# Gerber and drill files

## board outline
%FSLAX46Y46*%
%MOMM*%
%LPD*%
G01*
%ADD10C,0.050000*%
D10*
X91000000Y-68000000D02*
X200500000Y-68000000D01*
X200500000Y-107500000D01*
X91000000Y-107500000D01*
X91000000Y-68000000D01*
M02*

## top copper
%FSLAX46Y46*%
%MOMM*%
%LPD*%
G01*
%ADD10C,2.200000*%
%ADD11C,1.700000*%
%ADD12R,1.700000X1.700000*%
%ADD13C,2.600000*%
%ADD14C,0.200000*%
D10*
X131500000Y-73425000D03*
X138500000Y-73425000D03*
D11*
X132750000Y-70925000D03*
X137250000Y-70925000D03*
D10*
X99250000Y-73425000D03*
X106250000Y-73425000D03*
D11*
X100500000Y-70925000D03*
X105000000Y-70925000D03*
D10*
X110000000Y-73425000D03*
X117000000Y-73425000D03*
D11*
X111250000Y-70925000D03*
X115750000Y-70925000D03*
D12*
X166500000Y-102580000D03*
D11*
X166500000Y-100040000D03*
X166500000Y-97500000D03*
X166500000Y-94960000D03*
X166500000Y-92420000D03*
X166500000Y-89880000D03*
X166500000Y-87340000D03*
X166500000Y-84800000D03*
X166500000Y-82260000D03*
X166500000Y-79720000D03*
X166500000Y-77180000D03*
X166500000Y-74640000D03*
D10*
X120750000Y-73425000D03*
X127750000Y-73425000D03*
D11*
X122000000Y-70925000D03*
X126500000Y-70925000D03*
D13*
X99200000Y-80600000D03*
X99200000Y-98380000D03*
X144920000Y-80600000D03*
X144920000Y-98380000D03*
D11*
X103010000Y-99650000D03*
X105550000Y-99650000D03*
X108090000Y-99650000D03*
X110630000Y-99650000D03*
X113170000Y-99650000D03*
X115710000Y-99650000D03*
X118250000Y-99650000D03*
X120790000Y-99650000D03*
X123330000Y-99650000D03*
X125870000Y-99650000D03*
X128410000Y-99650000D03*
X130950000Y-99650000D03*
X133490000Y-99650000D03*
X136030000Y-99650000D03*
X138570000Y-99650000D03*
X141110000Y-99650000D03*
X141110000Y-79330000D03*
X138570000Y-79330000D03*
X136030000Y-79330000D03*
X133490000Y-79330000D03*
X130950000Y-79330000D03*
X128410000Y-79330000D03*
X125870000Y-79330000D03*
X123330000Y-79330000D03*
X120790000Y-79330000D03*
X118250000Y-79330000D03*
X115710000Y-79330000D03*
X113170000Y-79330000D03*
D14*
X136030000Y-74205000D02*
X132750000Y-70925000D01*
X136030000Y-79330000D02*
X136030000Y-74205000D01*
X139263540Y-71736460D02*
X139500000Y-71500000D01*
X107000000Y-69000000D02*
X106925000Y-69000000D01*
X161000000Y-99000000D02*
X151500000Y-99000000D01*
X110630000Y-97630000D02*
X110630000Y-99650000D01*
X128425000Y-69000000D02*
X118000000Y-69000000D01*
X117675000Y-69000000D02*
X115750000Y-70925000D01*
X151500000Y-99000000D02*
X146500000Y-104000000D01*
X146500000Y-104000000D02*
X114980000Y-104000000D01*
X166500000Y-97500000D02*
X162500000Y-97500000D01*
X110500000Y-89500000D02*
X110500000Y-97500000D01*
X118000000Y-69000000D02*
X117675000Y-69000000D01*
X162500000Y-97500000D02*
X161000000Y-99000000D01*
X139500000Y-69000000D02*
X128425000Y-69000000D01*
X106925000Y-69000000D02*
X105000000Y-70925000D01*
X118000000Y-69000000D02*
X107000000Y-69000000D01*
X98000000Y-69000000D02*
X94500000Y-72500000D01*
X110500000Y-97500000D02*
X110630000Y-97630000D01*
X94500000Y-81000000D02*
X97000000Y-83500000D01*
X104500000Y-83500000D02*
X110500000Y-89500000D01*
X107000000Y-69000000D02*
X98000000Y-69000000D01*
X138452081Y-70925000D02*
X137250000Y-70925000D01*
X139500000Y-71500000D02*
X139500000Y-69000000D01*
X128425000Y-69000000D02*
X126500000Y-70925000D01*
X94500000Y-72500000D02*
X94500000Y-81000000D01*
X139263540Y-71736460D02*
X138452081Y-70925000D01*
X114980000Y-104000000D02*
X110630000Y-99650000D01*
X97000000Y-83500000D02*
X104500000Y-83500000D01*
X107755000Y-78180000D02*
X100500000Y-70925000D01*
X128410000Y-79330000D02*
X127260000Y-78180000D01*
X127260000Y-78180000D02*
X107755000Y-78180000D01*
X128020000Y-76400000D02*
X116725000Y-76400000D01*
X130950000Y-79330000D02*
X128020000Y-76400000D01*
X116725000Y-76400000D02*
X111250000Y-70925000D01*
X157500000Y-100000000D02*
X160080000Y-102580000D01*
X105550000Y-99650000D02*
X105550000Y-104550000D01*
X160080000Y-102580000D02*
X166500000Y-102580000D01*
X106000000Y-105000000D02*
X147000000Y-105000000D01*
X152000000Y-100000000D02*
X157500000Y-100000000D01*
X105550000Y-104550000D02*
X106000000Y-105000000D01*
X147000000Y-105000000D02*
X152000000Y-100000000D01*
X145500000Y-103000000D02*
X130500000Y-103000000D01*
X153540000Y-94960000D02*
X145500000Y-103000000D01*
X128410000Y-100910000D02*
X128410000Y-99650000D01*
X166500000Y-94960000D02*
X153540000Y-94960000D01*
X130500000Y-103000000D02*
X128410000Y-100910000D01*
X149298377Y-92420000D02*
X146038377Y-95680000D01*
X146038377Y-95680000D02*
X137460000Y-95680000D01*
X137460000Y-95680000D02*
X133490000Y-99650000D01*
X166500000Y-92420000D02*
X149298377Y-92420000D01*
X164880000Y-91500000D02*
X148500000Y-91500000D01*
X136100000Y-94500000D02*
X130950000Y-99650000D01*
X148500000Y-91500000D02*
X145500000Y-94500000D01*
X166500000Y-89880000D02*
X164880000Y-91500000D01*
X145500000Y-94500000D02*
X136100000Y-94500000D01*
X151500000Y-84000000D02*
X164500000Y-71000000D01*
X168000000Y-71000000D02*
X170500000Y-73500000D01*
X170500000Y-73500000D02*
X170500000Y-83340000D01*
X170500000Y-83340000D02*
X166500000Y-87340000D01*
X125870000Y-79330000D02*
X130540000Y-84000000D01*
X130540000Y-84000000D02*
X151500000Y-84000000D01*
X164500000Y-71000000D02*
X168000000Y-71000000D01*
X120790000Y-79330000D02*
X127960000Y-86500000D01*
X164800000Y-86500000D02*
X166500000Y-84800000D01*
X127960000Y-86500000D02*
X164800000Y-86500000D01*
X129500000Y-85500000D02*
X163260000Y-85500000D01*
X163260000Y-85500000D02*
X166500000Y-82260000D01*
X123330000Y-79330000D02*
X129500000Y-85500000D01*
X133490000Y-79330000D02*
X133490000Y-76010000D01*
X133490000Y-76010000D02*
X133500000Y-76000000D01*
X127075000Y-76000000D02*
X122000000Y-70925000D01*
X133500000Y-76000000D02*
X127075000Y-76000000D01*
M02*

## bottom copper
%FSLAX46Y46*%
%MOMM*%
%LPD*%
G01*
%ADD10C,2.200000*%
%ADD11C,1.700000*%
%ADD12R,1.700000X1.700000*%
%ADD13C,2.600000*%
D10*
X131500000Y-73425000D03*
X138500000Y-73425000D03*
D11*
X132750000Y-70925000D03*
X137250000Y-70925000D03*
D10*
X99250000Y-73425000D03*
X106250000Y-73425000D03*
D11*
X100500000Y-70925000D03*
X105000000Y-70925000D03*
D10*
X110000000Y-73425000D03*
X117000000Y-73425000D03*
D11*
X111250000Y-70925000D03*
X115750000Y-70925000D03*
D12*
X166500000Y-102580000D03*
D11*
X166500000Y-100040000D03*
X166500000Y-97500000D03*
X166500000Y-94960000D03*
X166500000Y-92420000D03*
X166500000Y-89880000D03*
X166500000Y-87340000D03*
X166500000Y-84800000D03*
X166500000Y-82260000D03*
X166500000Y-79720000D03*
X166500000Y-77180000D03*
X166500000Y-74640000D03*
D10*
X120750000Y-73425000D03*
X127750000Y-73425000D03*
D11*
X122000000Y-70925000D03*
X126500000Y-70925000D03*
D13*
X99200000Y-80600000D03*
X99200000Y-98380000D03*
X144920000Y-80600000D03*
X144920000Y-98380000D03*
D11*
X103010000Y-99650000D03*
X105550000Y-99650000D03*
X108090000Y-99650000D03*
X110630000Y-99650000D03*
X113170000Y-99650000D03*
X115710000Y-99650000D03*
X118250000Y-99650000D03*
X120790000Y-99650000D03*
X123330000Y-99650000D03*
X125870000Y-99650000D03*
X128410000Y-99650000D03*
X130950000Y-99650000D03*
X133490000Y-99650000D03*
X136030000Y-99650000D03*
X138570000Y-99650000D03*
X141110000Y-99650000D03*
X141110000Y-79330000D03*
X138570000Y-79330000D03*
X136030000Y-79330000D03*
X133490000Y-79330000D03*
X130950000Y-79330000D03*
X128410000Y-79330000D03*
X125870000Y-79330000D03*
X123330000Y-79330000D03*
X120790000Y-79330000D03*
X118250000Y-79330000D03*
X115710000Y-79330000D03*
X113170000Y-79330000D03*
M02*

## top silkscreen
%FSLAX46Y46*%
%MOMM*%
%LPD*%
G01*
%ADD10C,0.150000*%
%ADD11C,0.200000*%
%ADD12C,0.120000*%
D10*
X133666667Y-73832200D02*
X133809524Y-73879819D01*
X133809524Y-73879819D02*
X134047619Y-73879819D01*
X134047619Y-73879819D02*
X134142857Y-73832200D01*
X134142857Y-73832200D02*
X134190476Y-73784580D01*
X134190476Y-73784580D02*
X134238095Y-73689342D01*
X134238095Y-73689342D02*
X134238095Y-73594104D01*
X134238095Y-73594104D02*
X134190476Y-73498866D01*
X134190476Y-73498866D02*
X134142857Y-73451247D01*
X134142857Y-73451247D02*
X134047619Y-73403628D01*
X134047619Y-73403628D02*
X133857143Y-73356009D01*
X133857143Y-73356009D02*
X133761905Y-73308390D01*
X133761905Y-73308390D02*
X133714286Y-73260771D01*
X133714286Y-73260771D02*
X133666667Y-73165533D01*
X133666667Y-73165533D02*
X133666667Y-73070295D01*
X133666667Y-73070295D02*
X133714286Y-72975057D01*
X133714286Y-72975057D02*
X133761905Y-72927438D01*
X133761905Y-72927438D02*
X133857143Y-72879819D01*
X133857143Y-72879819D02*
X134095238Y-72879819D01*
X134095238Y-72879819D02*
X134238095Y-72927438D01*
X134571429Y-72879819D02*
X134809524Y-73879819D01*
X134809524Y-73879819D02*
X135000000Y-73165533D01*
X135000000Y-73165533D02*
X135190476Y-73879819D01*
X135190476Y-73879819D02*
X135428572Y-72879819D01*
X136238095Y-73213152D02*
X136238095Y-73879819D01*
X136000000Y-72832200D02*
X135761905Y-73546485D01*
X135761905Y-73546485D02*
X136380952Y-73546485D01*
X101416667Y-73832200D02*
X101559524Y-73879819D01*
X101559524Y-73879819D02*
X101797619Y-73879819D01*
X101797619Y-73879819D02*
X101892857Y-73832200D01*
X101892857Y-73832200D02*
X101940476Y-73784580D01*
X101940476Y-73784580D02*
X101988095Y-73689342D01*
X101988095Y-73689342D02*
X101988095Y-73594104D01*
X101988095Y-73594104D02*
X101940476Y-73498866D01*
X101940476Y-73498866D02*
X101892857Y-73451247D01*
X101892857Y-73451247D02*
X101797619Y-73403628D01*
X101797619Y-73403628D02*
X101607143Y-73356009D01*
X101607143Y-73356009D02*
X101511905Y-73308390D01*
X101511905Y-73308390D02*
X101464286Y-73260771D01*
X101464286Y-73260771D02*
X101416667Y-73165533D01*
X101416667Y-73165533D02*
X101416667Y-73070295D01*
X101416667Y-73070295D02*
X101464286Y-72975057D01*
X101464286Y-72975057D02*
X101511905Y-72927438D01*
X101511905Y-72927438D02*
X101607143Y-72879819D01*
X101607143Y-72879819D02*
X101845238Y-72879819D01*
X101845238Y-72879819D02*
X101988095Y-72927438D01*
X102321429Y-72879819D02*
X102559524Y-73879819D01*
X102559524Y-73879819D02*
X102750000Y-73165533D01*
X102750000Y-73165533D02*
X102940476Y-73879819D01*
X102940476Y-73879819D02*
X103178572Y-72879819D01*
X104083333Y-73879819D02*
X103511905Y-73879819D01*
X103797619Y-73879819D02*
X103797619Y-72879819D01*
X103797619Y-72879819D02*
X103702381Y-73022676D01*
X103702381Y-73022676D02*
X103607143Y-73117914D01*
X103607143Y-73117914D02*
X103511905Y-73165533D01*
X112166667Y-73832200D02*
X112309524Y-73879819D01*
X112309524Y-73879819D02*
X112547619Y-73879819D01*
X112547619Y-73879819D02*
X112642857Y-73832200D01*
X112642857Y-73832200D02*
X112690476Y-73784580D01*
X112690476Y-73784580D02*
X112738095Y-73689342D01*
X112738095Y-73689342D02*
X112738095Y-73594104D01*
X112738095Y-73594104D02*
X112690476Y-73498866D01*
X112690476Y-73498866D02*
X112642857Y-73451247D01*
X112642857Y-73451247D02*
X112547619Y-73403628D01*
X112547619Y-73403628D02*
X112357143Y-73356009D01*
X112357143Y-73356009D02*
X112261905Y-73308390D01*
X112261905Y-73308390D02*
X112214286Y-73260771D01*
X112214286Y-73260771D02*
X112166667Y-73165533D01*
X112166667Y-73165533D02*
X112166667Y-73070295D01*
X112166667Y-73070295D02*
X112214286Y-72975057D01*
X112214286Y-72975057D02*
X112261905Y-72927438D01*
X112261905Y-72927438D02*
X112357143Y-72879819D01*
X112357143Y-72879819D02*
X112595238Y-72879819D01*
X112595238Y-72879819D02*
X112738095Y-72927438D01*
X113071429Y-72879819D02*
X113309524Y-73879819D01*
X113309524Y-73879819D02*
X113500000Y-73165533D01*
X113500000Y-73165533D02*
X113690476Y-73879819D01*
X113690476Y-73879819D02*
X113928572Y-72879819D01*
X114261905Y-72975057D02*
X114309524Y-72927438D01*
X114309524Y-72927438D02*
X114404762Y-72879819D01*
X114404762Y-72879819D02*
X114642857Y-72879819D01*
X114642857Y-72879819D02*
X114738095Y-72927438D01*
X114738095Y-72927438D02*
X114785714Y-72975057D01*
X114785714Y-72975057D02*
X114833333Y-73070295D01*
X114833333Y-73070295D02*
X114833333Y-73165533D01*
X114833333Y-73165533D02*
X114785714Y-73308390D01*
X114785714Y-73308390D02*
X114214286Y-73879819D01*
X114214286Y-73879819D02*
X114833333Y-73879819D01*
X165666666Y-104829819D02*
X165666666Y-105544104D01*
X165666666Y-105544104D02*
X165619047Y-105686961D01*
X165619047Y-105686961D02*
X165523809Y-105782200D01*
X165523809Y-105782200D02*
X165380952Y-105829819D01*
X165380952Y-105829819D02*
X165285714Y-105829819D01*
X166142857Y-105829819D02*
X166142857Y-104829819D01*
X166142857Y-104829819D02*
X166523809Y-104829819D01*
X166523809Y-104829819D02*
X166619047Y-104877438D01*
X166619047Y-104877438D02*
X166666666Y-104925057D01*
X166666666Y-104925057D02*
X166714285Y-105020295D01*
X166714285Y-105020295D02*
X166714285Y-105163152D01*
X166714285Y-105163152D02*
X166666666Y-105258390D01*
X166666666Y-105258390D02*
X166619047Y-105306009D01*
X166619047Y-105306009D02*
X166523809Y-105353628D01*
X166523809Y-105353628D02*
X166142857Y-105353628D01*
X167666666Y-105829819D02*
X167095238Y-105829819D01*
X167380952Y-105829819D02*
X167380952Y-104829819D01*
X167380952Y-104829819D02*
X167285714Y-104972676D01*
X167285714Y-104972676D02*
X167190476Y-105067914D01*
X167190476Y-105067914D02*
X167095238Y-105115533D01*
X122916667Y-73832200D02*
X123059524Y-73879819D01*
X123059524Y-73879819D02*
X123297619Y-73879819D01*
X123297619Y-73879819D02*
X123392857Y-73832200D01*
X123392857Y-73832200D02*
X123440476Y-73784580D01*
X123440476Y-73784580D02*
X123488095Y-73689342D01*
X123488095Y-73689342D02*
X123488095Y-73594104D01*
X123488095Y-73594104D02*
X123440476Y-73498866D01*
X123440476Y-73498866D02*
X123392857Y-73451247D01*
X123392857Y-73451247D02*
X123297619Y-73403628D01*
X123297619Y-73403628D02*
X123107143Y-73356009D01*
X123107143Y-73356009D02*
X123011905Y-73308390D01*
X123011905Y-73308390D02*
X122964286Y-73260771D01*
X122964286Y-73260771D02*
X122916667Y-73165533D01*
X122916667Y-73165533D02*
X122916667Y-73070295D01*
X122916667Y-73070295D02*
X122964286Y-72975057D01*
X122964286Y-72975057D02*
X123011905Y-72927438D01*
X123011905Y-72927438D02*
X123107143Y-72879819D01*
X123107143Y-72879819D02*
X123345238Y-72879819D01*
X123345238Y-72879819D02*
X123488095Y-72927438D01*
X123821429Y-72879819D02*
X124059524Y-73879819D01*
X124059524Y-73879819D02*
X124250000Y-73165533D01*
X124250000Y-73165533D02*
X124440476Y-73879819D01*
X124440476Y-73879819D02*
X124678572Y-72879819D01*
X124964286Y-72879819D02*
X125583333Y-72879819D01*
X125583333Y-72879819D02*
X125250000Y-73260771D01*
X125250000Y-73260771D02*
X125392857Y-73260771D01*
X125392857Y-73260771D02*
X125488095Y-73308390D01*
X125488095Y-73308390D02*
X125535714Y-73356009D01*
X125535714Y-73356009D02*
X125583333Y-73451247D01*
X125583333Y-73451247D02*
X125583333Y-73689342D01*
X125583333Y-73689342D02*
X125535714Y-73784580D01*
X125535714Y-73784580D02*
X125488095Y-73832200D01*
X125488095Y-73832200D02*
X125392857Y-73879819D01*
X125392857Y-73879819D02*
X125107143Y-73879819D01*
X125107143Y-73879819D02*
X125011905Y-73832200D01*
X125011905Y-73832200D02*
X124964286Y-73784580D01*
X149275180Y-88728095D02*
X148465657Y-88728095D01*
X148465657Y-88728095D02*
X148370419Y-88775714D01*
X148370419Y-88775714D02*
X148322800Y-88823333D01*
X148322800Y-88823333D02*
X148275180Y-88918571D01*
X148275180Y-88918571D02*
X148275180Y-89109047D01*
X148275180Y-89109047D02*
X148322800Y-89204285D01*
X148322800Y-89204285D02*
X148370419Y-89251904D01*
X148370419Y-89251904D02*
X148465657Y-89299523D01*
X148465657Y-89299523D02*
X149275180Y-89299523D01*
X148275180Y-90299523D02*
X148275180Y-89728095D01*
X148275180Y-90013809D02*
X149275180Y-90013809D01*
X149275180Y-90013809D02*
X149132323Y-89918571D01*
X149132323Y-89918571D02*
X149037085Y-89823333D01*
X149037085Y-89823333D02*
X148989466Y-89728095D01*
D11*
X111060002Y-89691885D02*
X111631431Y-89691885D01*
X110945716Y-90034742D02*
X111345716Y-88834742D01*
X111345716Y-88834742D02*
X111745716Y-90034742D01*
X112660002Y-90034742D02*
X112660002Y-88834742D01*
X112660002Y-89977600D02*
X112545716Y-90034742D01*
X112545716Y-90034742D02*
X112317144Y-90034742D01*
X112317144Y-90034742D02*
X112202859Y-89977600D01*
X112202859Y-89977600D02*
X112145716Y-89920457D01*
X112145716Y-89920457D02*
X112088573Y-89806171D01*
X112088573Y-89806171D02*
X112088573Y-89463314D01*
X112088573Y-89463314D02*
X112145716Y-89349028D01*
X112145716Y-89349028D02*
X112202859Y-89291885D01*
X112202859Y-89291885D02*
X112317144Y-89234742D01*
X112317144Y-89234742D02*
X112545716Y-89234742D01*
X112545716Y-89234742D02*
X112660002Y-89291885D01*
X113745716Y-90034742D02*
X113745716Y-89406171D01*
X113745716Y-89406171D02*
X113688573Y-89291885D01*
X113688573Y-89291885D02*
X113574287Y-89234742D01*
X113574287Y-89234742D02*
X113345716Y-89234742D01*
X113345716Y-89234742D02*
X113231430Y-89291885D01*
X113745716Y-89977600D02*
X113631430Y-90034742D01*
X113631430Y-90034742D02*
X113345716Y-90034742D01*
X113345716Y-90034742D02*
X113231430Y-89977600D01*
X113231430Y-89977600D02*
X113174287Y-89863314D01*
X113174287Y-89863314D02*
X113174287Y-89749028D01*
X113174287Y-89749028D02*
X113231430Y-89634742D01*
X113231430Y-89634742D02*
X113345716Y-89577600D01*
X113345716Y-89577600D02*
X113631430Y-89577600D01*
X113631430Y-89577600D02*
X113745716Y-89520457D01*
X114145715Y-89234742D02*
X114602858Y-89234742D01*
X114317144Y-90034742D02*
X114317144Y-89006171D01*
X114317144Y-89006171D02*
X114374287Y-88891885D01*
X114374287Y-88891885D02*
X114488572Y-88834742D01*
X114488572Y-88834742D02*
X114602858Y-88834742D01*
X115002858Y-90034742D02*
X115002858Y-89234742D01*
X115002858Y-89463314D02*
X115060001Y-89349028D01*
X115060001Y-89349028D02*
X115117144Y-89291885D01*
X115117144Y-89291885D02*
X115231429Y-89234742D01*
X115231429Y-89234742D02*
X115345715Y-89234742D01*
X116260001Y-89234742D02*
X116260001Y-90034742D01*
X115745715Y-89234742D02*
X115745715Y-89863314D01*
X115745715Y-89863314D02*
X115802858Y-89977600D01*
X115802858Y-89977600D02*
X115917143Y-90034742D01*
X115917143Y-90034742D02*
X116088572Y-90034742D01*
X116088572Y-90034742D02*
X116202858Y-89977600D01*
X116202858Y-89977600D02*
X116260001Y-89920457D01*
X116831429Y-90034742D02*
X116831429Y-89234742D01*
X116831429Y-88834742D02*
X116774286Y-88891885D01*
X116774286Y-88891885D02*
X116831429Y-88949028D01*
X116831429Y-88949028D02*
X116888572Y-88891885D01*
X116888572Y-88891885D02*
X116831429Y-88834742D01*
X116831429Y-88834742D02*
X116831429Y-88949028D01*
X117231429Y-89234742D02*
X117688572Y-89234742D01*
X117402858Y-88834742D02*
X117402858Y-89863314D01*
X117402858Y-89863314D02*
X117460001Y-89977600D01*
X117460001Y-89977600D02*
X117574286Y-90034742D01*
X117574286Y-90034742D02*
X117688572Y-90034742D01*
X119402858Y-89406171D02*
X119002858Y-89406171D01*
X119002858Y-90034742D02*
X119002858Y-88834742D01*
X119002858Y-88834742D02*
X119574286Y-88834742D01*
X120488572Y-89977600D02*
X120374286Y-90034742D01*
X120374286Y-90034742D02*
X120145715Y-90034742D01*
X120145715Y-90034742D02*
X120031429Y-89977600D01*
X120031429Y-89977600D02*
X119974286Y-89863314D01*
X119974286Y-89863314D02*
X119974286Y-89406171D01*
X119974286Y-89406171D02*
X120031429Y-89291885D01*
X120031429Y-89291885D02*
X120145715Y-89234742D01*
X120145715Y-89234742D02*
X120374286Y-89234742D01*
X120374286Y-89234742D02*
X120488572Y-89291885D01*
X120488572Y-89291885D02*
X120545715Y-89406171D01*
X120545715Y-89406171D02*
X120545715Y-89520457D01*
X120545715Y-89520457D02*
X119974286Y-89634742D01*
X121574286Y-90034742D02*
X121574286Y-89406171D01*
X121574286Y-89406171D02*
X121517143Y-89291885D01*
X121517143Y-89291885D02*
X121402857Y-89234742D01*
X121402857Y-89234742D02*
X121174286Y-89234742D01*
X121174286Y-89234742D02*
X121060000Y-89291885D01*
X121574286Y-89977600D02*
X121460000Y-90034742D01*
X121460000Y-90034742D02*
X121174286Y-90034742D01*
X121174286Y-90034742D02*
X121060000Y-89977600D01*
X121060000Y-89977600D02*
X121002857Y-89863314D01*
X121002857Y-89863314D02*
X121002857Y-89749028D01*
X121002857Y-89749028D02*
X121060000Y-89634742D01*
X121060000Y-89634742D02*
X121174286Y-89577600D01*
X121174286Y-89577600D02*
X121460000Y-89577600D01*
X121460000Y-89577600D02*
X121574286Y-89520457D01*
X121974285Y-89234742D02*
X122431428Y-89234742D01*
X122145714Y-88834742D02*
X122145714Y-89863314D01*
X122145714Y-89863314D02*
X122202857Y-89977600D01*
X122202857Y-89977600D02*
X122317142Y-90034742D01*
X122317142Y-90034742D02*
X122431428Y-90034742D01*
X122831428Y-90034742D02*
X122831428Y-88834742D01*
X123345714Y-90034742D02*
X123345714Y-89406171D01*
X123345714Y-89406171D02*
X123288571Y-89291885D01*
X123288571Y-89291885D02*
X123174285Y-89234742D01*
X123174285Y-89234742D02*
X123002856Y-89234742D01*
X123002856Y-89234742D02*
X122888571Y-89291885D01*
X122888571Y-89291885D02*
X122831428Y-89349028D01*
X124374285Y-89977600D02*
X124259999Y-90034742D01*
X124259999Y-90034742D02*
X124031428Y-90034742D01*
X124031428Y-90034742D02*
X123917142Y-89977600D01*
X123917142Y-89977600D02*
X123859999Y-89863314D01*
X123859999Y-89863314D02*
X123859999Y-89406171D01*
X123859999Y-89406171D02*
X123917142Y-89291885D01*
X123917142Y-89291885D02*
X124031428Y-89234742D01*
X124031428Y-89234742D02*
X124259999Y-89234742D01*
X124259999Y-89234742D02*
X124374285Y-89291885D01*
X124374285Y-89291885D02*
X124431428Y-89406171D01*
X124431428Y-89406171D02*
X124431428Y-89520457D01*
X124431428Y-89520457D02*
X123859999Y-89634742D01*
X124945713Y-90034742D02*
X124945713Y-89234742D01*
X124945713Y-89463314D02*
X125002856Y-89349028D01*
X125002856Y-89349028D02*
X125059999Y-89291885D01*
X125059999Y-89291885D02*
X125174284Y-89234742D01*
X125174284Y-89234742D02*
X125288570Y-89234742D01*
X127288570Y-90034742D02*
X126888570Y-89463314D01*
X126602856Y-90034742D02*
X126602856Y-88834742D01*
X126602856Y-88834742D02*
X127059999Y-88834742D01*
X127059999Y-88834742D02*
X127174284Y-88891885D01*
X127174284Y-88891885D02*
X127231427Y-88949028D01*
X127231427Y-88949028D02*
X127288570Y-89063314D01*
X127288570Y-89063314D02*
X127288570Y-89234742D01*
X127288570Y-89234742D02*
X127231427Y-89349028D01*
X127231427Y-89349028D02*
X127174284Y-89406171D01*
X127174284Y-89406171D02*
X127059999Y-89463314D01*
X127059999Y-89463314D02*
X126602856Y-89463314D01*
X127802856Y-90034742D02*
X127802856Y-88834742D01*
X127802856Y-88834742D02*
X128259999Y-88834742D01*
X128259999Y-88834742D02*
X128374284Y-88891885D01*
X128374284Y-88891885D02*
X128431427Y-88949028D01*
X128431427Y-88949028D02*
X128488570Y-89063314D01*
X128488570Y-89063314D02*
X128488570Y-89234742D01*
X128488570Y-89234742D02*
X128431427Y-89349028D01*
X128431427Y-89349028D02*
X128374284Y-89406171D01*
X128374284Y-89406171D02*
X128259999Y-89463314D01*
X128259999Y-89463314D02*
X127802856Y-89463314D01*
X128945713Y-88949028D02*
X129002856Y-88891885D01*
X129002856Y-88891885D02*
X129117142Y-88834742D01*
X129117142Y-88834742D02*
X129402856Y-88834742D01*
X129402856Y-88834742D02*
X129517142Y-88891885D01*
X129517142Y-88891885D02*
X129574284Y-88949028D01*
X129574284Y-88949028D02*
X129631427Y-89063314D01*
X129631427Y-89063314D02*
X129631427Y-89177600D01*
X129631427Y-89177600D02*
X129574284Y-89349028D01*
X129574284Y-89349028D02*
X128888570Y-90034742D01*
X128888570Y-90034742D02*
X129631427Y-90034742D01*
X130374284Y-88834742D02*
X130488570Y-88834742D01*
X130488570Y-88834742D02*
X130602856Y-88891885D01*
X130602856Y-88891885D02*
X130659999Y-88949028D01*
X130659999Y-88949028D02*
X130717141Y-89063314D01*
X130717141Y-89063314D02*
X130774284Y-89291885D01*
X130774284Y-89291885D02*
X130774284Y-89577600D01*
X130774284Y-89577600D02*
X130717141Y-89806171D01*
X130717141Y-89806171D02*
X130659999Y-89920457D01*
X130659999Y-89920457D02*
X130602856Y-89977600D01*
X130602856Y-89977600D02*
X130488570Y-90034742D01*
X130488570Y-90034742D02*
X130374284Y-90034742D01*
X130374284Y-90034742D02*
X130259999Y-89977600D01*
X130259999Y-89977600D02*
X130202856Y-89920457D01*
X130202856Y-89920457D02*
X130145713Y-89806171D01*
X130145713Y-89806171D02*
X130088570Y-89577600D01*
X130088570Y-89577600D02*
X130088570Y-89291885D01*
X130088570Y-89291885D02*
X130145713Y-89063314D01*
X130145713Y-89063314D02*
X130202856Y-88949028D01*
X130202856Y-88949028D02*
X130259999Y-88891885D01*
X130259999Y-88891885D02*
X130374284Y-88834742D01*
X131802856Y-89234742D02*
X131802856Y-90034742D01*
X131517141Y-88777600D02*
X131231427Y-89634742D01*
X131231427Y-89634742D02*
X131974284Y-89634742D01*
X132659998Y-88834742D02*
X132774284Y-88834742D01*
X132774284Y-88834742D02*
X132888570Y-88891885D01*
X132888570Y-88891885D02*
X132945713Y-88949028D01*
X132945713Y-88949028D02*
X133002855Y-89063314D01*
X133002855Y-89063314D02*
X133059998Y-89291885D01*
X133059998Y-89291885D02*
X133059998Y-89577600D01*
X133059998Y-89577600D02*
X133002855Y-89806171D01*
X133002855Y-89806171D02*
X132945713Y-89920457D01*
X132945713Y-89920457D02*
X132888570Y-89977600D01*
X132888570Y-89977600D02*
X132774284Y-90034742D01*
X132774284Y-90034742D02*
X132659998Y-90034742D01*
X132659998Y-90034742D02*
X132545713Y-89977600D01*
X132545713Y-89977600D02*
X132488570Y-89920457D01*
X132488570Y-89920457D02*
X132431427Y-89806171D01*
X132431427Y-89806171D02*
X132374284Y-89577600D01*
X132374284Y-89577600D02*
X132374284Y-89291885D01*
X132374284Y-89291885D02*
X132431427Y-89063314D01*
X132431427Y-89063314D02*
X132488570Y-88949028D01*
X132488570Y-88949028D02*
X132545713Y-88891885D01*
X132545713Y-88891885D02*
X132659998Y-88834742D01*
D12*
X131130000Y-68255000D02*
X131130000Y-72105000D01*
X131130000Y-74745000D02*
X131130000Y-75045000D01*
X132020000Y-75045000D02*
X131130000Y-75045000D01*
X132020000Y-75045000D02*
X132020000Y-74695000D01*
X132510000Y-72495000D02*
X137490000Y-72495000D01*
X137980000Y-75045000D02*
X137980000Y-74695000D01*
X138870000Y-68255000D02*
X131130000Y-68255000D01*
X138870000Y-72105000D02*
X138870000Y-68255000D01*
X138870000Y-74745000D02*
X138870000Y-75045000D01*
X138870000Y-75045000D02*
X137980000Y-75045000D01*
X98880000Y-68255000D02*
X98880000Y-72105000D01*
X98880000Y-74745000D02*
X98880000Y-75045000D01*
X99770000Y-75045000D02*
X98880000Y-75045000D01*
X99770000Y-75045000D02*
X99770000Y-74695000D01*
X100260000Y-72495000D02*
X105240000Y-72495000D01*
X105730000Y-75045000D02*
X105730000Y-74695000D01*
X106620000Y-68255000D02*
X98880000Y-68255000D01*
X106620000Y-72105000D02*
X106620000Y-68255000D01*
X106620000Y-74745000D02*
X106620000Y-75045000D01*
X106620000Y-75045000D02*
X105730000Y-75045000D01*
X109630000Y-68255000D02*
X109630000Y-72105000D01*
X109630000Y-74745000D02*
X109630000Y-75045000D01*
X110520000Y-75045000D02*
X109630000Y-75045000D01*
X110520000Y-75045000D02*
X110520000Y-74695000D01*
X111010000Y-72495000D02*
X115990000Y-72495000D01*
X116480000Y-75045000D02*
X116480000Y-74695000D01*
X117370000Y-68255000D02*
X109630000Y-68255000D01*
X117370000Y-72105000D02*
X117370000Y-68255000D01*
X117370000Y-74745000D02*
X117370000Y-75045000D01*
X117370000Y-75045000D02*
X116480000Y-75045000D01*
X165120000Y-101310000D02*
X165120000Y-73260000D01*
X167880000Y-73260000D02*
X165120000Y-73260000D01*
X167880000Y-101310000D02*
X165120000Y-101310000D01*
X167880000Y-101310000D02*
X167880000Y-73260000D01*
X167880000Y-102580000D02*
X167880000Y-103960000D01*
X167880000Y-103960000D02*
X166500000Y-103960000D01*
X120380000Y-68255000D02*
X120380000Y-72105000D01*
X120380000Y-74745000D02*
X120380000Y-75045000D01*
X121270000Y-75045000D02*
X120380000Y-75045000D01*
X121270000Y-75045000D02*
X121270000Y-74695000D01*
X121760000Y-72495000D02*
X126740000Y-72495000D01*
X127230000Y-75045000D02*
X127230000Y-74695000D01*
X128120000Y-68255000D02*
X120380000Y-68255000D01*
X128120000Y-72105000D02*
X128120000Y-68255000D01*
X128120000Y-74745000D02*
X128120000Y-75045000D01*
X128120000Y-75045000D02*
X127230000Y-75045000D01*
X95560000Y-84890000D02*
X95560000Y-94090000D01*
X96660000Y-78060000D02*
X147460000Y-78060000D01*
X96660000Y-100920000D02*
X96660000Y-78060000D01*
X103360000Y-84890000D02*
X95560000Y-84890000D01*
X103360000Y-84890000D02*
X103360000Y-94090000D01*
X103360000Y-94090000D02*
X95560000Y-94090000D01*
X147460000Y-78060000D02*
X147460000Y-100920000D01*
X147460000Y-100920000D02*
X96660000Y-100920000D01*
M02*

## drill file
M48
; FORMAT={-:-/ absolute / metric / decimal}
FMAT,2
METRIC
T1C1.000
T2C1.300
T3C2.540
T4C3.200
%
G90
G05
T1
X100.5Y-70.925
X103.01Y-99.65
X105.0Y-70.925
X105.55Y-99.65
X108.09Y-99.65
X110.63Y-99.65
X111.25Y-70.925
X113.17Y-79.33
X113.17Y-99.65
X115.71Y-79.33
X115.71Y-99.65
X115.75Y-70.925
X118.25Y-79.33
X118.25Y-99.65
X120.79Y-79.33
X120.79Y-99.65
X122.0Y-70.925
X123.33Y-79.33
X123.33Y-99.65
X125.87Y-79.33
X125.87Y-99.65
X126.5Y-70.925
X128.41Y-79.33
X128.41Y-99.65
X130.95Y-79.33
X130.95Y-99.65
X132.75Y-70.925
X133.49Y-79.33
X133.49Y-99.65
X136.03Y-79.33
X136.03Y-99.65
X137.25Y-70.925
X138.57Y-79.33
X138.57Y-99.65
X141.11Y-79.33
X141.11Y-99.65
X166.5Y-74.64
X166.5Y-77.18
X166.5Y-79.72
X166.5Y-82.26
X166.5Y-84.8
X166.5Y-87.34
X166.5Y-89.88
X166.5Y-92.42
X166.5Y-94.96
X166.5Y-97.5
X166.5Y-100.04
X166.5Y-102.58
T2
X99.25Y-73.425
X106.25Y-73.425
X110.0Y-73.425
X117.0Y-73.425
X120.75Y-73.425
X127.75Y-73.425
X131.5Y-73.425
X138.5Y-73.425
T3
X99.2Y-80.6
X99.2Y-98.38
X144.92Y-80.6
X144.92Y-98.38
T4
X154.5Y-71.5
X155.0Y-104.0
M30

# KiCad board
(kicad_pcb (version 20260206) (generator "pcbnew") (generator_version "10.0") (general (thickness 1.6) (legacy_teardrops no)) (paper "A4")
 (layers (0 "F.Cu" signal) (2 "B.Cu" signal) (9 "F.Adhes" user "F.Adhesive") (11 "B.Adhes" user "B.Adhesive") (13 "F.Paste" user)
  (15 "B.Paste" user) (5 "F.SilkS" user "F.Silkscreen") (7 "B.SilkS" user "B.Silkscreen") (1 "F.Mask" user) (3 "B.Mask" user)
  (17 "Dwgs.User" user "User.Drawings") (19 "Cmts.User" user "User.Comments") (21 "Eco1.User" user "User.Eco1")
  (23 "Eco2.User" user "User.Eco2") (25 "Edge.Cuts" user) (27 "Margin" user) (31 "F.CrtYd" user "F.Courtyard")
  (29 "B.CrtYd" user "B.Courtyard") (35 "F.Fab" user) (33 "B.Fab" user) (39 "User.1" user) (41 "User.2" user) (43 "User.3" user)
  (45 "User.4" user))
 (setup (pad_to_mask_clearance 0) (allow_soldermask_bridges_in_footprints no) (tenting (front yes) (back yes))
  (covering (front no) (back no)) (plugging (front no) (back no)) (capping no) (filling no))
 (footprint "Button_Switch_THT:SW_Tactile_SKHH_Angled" (layer "F.Cu") (at 132.75 70.925)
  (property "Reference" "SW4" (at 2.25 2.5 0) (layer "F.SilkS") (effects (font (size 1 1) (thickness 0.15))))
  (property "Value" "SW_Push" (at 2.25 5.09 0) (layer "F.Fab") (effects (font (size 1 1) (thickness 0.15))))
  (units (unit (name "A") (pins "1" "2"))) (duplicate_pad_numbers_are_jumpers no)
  (fp_line (start -1.62 -2.67) (end -1.62 1.18) (stroke (width 0.12) (type solid)) (layer "F.SilkS"))
  (fp_line (start -1.62 3.82) (end -1.62 4.12) (stroke (width 0.12) (type solid)) (layer "F.SilkS"))
  (fp_line (start -0.73 4.12) (end -1.62 4.12) (stroke (width 0.12) (type solid)) (layer "F.SilkS"))
  (fp_line (start -0.73 4.12) (end -0.73 3.77) (stroke (width 0.12) (type solid)) (layer "F.SilkS"))
  (fp_line (start -0.24 1.57) (end 4.74 1.57) (stroke (width 0.12) (type solid)) (layer "F.SilkS"))
  (fp_line (start 5.23 4.12) (end 5.23 3.77) (stroke (width 0.12) (type solid)) (layer "F.SilkS"))
  (fp_line (start 6.12 -2.67) (end -1.62 -2.67) (stroke (width 0.12) (type solid)) (layer "F.SilkS"))
  (fp_line (start 6.12 1.18) (end 6.12 -2.67) (stroke (width 0.12) (type solid)) (layer "F.SilkS"))
  (fp_line (start 6.12 3.82) (end 6.12 4.12) (stroke (width 0.12) (type solid)) (layer "F.SilkS"))
  (fp_line (start 6.12 4.12) (end 5.23 4.12) (stroke (width 0.12) (type solid)) (layer "F.SilkS"))
  (pad "" thru_hole circle (at -1.25 2.5 180) (size 2.2 2.2) (drill 1.3) (layers "*.Cu" "*.Mask") (remove_unused_layers no))
  (pad "" thru_hole circle (at 5.75 2.5 180) (size 2.2 2.2) (drill 1.3) (layers "*.Cu" "*.Mask") (remove_unused_layers no))
  (pad "1" thru_hole circle (at 0 0 180) (size 1.7 1.7) (drill 1) (layers "*.Cu" "*.Mask") (remove_unused_layers no)
   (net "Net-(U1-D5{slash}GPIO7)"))
  (pad "2" thru_hole circle (at 4.5 0 180) (size 1.7 1.7) (drill 1) (layers "*.Cu" "*.Mask") (remove_unused_layers no) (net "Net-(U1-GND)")))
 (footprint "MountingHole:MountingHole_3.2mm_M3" (layer "F.Cu") (at 155 104)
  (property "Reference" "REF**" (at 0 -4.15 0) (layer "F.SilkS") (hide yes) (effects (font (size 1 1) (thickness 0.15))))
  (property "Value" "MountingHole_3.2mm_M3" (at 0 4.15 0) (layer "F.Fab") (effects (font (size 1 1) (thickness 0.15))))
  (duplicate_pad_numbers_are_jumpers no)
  (pad "" np_thru_hole circle (at 0 0) (size 3.2 3.2) (drill 3.2) (layers "*.Cu" "*.Mask")))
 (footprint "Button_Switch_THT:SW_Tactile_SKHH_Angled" (layer "F.Cu") (at 100.5 70.925)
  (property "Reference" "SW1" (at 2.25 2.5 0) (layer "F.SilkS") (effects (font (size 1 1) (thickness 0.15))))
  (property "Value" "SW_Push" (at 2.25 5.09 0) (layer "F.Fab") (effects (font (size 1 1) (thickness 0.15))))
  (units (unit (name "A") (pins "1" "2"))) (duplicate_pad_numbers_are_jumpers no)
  (fp_line (start -1.62 -2.67) (end -1.62 1.18) (stroke (width 0.12) (type solid)) (layer "F.SilkS"))
  (fp_line (start -1.62 3.82) (end -1.62 4.12) (stroke (width 0.12) (type solid)) (layer "F.SilkS"))
  (fp_line (start -0.73 4.12) (end -1.62 4.12) (stroke (width 0.12) (type solid)) (layer "F.SilkS"))
  (fp_line (start -0.73 4.12) (end -0.73 3.77) (stroke (width 0.12) (type solid)) (layer "F.SilkS"))
  (fp_line (start -0.24 1.57) (end 4.74 1.57) (stroke (width 0.12) (type solid)) (layer "F.SilkS"))
  (fp_line (start 5.23 4.12) (end 5.23 3.77) (stroke (width 0.12) (type solid)) (layer "F.SilkS"))
  (fp_line (start 6.12 -2.67) (end -1.62 -2.67) (stroke (width 0.12) (type solid)) (layer "F.SilkS"))
  (fp_line (start 6.12 1.18) (end 6.12 -2.67) (stroke (width 0.12) (type solid)) (layer "F.SilkS"))
  (fp_line (start 6.12 3.82) (end 6.12 4.12) (stroke (width 0.12) (type solid)) (layer "F.SilkS"))
  (fp_line (start 6.12 4.12) (end 5.23 4.12) (stroke (width 0.12) (type solid)) (layer "F.SilkS"))
  (pad "" thru_hole circle (at -1.25 2.5 180) (size 2.2 2.2) (drill 1.3) (layers "*.Cu" "*.Mask") (remove_unused_layers no))
  (pad "" thru_hole circle (at 5.75 2.5 180) (size 2.2 2.2) (drill 1.3) (layers "*.Cu" "*.Mask") (remove_unused_layers no))
  (pad "1" thru_hole circle (at 0 0 180) (size 1.7 1.7) (drill 1) (layers "*.Cu" "*.Mask") (remove_unused_layers no)
   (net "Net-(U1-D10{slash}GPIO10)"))
  (pad "2" thru_hole circle (at 4.5 0 180) (size 1.7 1.7) (drill 1) (layers "*.Cu" "*.Mask") (remove_unused_layers no) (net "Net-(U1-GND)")))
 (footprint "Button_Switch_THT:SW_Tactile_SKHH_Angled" (layer "F.Cu") (at 111.25 70.925)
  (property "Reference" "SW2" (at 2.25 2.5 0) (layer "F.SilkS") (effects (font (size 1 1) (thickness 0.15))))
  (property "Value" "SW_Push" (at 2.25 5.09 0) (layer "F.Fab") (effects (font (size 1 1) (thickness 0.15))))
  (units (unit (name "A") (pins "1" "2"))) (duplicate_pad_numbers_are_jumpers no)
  (fp_line (start -1.62 -2.67) (end -1.62 1.18) (stroke (width 0.12) (type solid)) (layer "F.SilkS"))
  (fp_line (start -1.62 3.82) (end -1.62 4.12) (stroke (width 0.12) (type solid)) (layer "F.SilkS"))
  (fp_line (start -0.73 4.12) (end -1.62 4.12) (stroke (width 0.12) (type solid)) (layer "F.SilkS"))
  (fp_line (start -0.73 4.12) (end -0.73 3.77) (stroke (width 0.12) (type solid)) (layer "F.SilkS"))
  (fp_line (start -0.24 1.57) (end 4.74 1.57) (stroke (width 0.12) (type solid)) (layer "F.SilkS"))
  (fp_line (start 5.23 4.12) (end 5.23 3.77) (stroke (width 0.12) (type solid)) (layer "F.SilkS"))
  (fp_line (start 6.12 -2.67) (end -1.62 -2.67) (stroke (width 0.12) (type solid)) (layer "F.SilkS"))
  (fp_line (start 6.12 1.18) (end 6.12 -2.67) (stroke (width 0.12) (type solid)) (layer "F.SilkS"))
  (fp_line (start 6.12 3.82) (end 6.12 4.12) (stroke (width 0.12) (type solid)) (layer "F.SilkS"))
  (fp_line (start 6.12 4.12) (end 5.23 4.12) (stroke (width 0.12) (type solid)) (layer "F.SilkS"))
  (pad "" thru_hole circle (at -1.25 2.5 180) (size 2.2 2.2) (drill 1.3) (layers "*.Cu" "*.Mask") (remove_unused_layers no))
  (pad "" thru_hole circle (at 5.75 2.5 180) (size 2.2 2.2) (drill 1.3) (layers "*.Cu" "*.Mask") (remove_unused_layers no))
  (pad "1" thru_hole circle (at 0 0 180) (size 1.7 1.7) (drill 1) (layers "*.Cu" "*.Mask") (remove_unused_layers no)
   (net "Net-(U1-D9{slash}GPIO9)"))
  (pad "2" thru_hole circle (at 4.5 0 180) (size 1.7 1.7) (drill 1) (layers "*.Cu" "*.Mask") (remove_unused_layers no) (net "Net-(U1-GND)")))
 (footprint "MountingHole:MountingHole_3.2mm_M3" (layer "F.Cu") (at 154.5 71.5)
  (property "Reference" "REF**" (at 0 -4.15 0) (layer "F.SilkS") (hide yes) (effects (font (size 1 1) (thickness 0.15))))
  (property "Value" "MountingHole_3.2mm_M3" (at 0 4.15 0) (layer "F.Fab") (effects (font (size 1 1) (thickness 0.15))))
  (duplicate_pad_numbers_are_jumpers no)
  (pad "" np_thru_hole circle (at 0 0) (size 3.2 3.2) (drill 3.2) (layers "*.Cu" "*.Mask")))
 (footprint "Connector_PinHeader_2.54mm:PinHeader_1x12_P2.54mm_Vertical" (layer "F.Cu") (at 166.5 102.58 180)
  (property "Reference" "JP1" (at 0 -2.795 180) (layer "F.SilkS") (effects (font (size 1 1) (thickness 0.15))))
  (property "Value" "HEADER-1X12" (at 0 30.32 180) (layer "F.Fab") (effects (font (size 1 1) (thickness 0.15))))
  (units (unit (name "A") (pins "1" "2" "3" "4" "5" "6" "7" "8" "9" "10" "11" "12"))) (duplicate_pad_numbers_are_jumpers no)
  (fp_line (start 1.38 1.27) (end 1.38 29.32) (stroke (width 0.12) (type solid)) (layer "F.SilkS"))
  (fp_line (start -1.38 29.32) (end 1.38 29.32) (stroke (width 0.12) (type solid)) (layer "F.SilkS"))
  (fp_line (start -1.38 1.27) (end 1.38 1.27) (stroke (width 0.12) (type solid)) (layer "F.SilkS"))
  (fp_line (start -1.38 1.27) (end -1.38 29.32) (stroke (width 0.12) (type solid)) (layer "F.SilkS"))
  (fp_line (start -1.38 0) (end -1.38 -1.38) (stroke (width 0.12) (type solid)) (layer "F.SilkS"))
  (fp_line (start -1.38 -1.38) (end 0 -1.38) (stroke (width 0.12) (type solid)) (layer "F.SilkS"))
  (pad "1" thru_hole rect (at 0 0 180) (size 1.7 1.7) (drill 1) (layers "*.Cu" "*.Mask") (remove_unused_layers no) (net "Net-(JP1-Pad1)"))
  (pad "2" thru_hole circle (at 0 2.54 180) (size 1.7 1.7) (drill 1) (layers "*.Cu" "*.Mask") (remove_unused_layers no)
   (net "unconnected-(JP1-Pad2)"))
  (pad "3" thru_hole circle (at 0 5.08 180) (size 1.7 1.7) (drill 1) (layers "*.Cu" "*.Mask") (remove_unused_layers no) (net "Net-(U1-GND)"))
  (pad "4" thru_hole circle (at 0 7.62 180) (size 1.7 1.7) (drill 1) (layers "*.Cu" "*.Mask") (remove_unused_layers no) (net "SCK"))
  (pad "5" thru_hole circle (at 0 10.16 180) (size 1.7 1.7) (drill 1) (layers "*.Cu" "*.Mask") (remove_unused_layers no) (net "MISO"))
  (pad "6" thru_hole circle (at 0 12.7 180) (size 1.7 1.7) (drill 1) (layers "*.Cu" "*.Mask") (remove_unused_layers no) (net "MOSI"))
  (pad "7" thru_hole circle (at 0 15.24 180) (size 1.7 1.7) (drill 1) (layers "*.Cu" "*.Mask") (remove_unused_layers no) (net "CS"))
  (pad "8" thru_hole circle (at 0 17.78 180) (size 1.7 1.7) (drill 1) (layers "*.Cu" "*.Mask") (remove_unused_layers no) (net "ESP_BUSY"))
  (pad "9" thru_hole circle (at 0 20.32 180) (size 1.7 1.7) (drill 1) (layers "*.Cu" "*.Mask") (remove_unused_layers no) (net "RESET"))
  (pad "10" thru_hole circle (at 0 22.86 180) (size 1.7 1.7) (drill 1) (layers "*.Cu" "*.Mask") (remove_unused_layers no) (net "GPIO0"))
  (pad "11" thru_hole circle (at 0 25.4 180) (size 1.7 1.7) (drill 1) (layers "*.Cu" "*.Mask") (remove_unused_layers no) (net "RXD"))
  (pad "12" thru_hole circle (at 0 27.94 180) (size 1.7 1.7) (drill 1) (layers "*.Cu" "*.Mask") (remove_unused_layers no) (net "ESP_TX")))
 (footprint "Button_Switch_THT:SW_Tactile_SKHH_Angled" (layer "F.Cu") (at 122 70.925)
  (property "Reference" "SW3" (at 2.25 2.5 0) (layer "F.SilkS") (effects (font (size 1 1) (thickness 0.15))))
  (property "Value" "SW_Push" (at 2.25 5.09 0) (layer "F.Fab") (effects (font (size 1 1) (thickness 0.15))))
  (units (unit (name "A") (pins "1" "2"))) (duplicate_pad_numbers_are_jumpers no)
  (fp_line (start -1.62 -2.67) (end -1.62 1.18) (stroke (width 0.12) (type solid)) (layer "F.SilkS"))
  (fp_line (start -1.62 3.82) (end -1.62 4.12) (stroke (width 0.12) (type solid)) (layer "F.SilkS"))
  (fp_line (start -0.73 4.12) (end -1.62 4.12) (stroke (width 0.12) (type solid)) (layer "F.SilkS"))
  (fp_line (start -0.73 4.12) (end -0.73 3.77) (stroke (width 0.12) (type solid)) (layer "F.SilkS"))
  (fp_line (start -0.24 1.57) (end 4.74 1.57) (stroke (width 0.12) (type solid)) (layer "F.SilkS"))
  (fp_line (start 5.23 4.12) (end 5.23 3.77) (stroke (width 0.12) (type solid)) (layer "F.SilkS"))
  (fp_line (start 6.12 -2.67) (end -1.62 -2.67) (stroke (width 0.12) (type solid)) (layer "F.SilkS"))
  (fp_line (start 6.12 1.18) (end 6.12 -2.67) (stroke (width 0.12) (type solid)) (layer "F.SilkS"))
  (fp_line (start 6.12 3.82) (end 6.12 4.12) (stroke (width 0.12) (type solid)) (layer "F.SilkS"))
  (fp_line (start 6.12 4.12) (end 5.23 4.12) (stroke (width 0.12) (type solid)) (layer "F.SilkS"))
  (pad "" thru_hole circle (at -1.25 2.5 180) (size 2.2 2.2) (drill 1.3) (layers "*.Cu" "*.Mask") (remove_unused_layers no))
  (pad "" thru_hole circle (at 5.75 2.5 180) (size 2.2 2.2) (drill 1.3) (layers "*.Cu" "*.Mask") (remove_unused_layers no))
  (pad "1" thru_hole circle (at 0 0 180) (size 1.7 1.7) (drill 1) (layers "*.Cu" "*.Mask") (remove_unused_layers no)
   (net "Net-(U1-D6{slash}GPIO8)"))
  (pad "2" thru_hole circle (at 4.5 0 180) (size 1.7 1.7) (drill 1) (layers "*.Cu" "*.Mask") (remove_unused_layers no) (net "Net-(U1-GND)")))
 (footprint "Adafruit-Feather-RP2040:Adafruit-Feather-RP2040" (layer "F.Cu") (at 122.06 89.49)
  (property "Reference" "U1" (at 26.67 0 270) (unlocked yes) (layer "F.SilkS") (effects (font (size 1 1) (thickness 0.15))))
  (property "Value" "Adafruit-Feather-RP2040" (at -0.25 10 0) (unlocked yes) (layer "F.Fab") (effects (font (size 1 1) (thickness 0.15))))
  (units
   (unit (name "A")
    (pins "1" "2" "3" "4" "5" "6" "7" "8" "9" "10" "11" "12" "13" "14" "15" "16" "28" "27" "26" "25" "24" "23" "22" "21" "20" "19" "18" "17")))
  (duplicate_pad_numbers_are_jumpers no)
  (fp_line (start -26.5 -4.6) (end -26.5 4.6) (stroke (width 0.12) (type solid)) (layer "F.SilkS"))
  (fp_line (start -25.4 -11.43) (end 25.4 -11.43) (stroke (width 0.12) (type solid)) (layer "F.SilkS"))
  (fp_line (start -25.4 11.43) (end -25.4 -11.43) (stroke (width 0.12) (type solid)) (layer "F.SilkS"))
  (fp_line (start -18.7 -4.6) (end -26.5 -4.6) (stroke (width 0.12) (type solid)) (layer "F.SilkS"))
  (fp_line (start -18.7 -4.6) (end -18.7 4.6) (stroke (width 0.12) (type solid)) (layer "F.SilkS"))
  (fp_line (start -18.7 4.6) (end -26.5 4.6) (stroke (width 0.12) (type solid)) (layer "F.SilkS"))
  (fp_line (start 25.4 -11.43) (end 25.4 11.43) (stroke (width 0.12) (type solid)) (layer "F.SilkS"))
  (fp_line (start 25.4 11.43) (end -25.4 11.43) (stroke (width 0.12) (type solid)) (layer "F.SilkS"))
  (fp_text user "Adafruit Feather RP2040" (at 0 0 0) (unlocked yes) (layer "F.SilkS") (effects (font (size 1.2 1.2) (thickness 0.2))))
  (pad "" np_thru_hole circle (at -22.86 -8.89) (size 2.6 2.6) (drill 2.54) (layers "*.Cu" "*.Mask") (solder_mask_margin 1.3)
   (clearance 1.3))
  (pad "" np_thru_hole circle (at -22.86 8.89) (size 2.6 2.6) (drill 2.54) (layers "*.Cu" "*.Mask") (solder_mask_margin 1.3) (clearance 1.3))
  (pad "" np_thru_hole circle (at 22.86 -8.89) (size 2.6 2.6) (drill 2.54) (layers "*.Cu" "*.Mask") (solder_mask_margin 1.3) (clearance 1.3))
  (pad "" np_thru_hole circle (at 22.86 8.89) (size 2.6 2.6) (drill 2.54) (layers "*.Cu" "*.Mask") (solder_mask_margin 1.3) (clearance 1.3))
  (pad "1" thru_hole circle (at -19.05 10.16) (size 1.7 1.7) (drill 1) (layers "*.Cu" "*.Mask") (remove_unused_layers no)
   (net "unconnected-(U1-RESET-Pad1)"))
  (pad "2" thru_hole circle (at -16.51 10.16) (size 1.7 1.7) (drill 1) (layers "*.Cu" "*.Mask") (remove_unused_layers no)
   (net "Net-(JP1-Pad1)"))
  (pad "3" thru_hole circle (at -13.97 10.16) (size 1.7 1.7) (drill 1) (layers "*.Cu" "*.Mask") (remove_unused_layers no)
   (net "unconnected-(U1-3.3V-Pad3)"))
  (pad "4" thru_hole circle (at -11.43 10.16) (size 1.7 1.7) (drill 1) (layers "*.Cu" "*.Mask") (remove_unused_layers no)
   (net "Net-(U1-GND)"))
  (pad "5" thru_hole circle (at -8.89 10.16) (size 1.7 1.7) (drill 1) (layers "*.Cu" "*.Mask") (remove_unused_layers no)
   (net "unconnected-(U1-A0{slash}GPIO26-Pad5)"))
  (pad "6" thru_hole circle (at -6.35 10.16) (size 1.7 1.7) (drill 1) (layers "*.Cu" "*.Mask") (remove_unused_layers no)
   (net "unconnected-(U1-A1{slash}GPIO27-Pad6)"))
  (pad "7" thru_hole circle (at -3.81 10.16) (size 1.7 1.7) (drill 1) (layers "*.Cu" "*.Mask") (remove_unused_layers no)
   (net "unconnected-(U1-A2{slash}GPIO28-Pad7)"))
  (pad "8" thru_hole circle (at -1.27 10.16) (size 1.7 1.7) (drill 1) (layers "*.Cu" "*.Mask") (remove_unused_layers no)
   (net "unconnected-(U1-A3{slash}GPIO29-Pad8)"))
  (pad "9" thru_hole circle (at 1.27 10.16) (size 1.7 1.7) (drill 1) (layers "*.Cu" "*.Mask") (remove_unused_layers no)
   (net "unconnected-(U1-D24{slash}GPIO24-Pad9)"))
  (pad "10" thru_hole circle (at 3.81 10.16) (size 1.7 1.7) (drill 1) (layers "*.Cu" "*.Mask") (remove_unused_layers no)
   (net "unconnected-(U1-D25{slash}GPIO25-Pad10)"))
  (pad "11" thru_hole circle (at 6.35 10.16) (size 1.7 1.7) (drill 1) (layers "*.Cu" "*.Mask") (remove_unused_layers no) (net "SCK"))
  (pad "12" thru_hole circle (at 8.89 10.16) (size 1.7 1.7) (drill 1) (layers "*.Cu" "*.Mask") (remove_unused_layers no) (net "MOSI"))
  (pad "13" thru_hole circle (at 11.43 10.16) (size 1.7 1.7) (drill 1) (layers "*.Cu" "*.Mask") (remove_unused_layers no) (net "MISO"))
  (pad "14" thru_hole circle (at 13.97 10.16) (size 1.7 1.7) (drill 1) (layers "*.Cu" "*.Mask") (remove_unused_layers no)
   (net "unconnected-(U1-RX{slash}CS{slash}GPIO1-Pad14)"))
  (pad "15" thru_hole circle (at 16.51 10.16) (size 1.7 1.7) (drill 1) (layers "*.Cu" "*.Mask") (remove_unused_layers no)
   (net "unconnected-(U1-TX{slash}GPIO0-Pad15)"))
  (pad "16" thru_hole circle (at 19.05 10.16) (size 1.7 1.7) (drill 1) (layers "*.Cu" "*.Mask") (remove_unused_layers no)
   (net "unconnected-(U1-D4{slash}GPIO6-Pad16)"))
  (pad "17" thru_hole circle (at 19.05 -10.16) (size 1.7 1.7) (drill 1) (layers "*.Cu" "*.Mask") (remove_unused_layers no)
   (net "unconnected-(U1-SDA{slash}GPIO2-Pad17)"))
  (pad "18" thru_hole circle (at 16.51 -10.16) (size 1.7 1.7) (drill 1) (layers "*.Cu" "*.Mask") (remove_unused_layers no)
   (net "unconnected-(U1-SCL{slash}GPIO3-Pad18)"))
  (pad "19" thru_hole circle (at 13.97 -10.16) (size 1.7 1.7) (drill 1) (layers "*.Cu" "*.Mask") (remove_unused_layers no)
   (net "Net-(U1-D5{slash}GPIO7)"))
  (pad "20" thru_hole circle (at 11.43 -10.16) (size 1.7 1.7) (drill 1) (layers "*.Cu" "*.Mask") (remove_unused_layers no)
   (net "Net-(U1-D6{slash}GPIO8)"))
  (pad "21" thru_hole circle (at 8.89 -10.16) (size 1.7 1.7) (drill 1) (layers "*.Cu" "*.Mask") (remove_unused_layers no)
   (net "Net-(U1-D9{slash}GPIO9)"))
  (pad "22" thru_hole circle (at 6.35 -10.16) (size 1.7 1.7) (drill 1) (layers "*.Cu" "*.Mask") (remove_unused_layers no)
   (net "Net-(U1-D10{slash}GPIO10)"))
  (pad "23" thru_hole circle (at 3.81 -10.16) (size 1.7 1.7) (drill 1) (layers "*.Cu" "*.Mask") (remove_unused_layers no) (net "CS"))
  (pad "24" thru_hole circle (at 1.27 -10.16) (size 1.7 1.7) (drill 1) (layers "*.Cu" "*.Mask") (remove_unused_layers no) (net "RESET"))
  (pad "25" thru_hole circle (at -1.27 -10.16) (size 1.7 1.7) (drill 1) (layers "*.Cu" "*.Mask") (remove_unused_layers no) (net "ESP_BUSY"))
  (pad "26" thru_hole circle (at -3.81 -10.16) (size 1.7 1.7) (drill 1) (layers "*.Cu" "*.Mask") (remove_unused_layers no)
   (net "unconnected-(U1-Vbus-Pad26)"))
  (pad "27" thru_hole circle (at -6.35 -10.16) (size 1.7 1.7) (drill 1) (layers "*.Cu" "*.Mask") (remove_unused_layers no)
   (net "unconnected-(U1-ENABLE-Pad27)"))
  (pad "28" thru_hole circle (at -8.89 -10.16) (size 1.7 1.7) (drill 1) (layers "*.Cu" "*.Mask") (remove_unused_layers no)
   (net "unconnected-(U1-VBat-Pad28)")))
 (gr_rect (start 91 68) (end 200.5 107.5) (stroke (width 0.05) (type default)) (fill no) (layer "Edge.Cuts"))
 (segment (start 136.03 74.205) (end 132.75 70.925) (width 0.2) (layer "F.Cu") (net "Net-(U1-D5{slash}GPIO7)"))
 (segment (start 136.03 79.33) (end 136.03 74.205) (width 0.2) (layer "F.Cu") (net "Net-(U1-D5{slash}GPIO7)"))
 (segment (start 139.26354 71.73646) (end 139.5 71.5) (width 0.2) (layer "F.Cu") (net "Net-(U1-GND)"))
 (segment (start 107 69) (end 106.925 69) (width 0.2) (layer "F.Cu") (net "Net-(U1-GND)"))
 (segment (start 161 99) (end 151.5 99) (width 0.2) (layer "F.Cu") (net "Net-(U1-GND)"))
 (segment (start 110.63 97.63) (end 110.63 99.65) (width 0.2) (layer "F.Cu") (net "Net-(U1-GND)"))
 (segment (start 128.425 69) (end 118 69) (width 0.2) (layer "F.Cu") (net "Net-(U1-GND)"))
 (segment (start 117.675 69) (end 115.75 70.925) (width 0.2) (layer "F.Cu") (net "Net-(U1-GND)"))
 (segment (start 151.5 99) (end 146.5 104) (width 0.2) (layer "F.Cu") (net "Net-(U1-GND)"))
 (segment (start 146.5 104) (end 114.98 104) (width 0.2) (layer "F.Cu") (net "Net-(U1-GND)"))
 (segment (start 166.5 97.5) (end 162.5 97.5) (width 0.2) (layer "F.Cu") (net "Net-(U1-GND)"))
 (segment (start 110.5 89.5) (end 110.5 97.5) (width 0.2) (layer "F.Cu") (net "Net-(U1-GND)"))
 (segment (start 118 69) (end 117.675 69) (width 0.2) (layer "F.Cu") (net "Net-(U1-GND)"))
 (segment (start 162.5 97.5) (end 161 99) (width 0.2) (layer "F.Cu") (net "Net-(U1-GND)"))
 (segment (start 139.5 69) (end 128.425 69) (width 0.2) (layer "F.Cu") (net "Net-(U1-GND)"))
 (segment (start 106.925 69) (end 105 70.925) (width 0.2) (layer "F.Cu") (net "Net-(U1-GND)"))
 (segment (start 118 69) (end 107 69) (width 0.2) (layer "F.Cu") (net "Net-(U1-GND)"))
 (segment (start 98 69) (end 94.5 72.5) (width 0.2) (layer "F.Cu") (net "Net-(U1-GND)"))
 (segment (start 110.5 97.5) (end 110.63 97.63) (width 0.2) (layer "F.Cu") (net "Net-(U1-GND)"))
 (segment (start 94.5 81) (end 97 83.5) (width 0.2) (layer "F.Cu") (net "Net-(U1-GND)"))
 (segment (start 104.5 83.5) (end 110.5 89.5) (width 0.2) (layer "F.Cu") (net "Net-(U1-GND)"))
 (segment (start 107 69) (end 98 69) (width 0.2) (layer "F.Cu") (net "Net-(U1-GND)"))
 (segment (start 138.452081 70.925) (end 137.25 70.925) (width 0.2) (layer "F.Cu") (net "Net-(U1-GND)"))
 (segment (start 139.5 71.5) (end 139.5 69) (width 0.2) (layer "F.Cu") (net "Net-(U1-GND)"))
 (segment (start 128.425 69) (end 126.5 70.925) (width 0.2) (layer "F.Cu") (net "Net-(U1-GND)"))
 (segment (start 94.5 72.5) (end 94.5 81) (width 0.2) (layer "F.Cu") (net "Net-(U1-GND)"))
 (segment (start 139.26354 71.73646) (end 138.452081 70.925) (width 0.2) (layer "F.Cu") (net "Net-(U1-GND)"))
 (segment (start 114.98 104) (end 110.63 99.65) (width 0.2) (layer "F.Cu") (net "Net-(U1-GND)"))
 (segment (start 97 83.5) (end 104.5 83.5) (width 0.2) (layer "F.Cu") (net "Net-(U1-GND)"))
 (segment (start 107.755 78.18) (end 100.5 70.925) (width 0.2) (layer "F.Cu") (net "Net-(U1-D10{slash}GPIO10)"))
 (segment (start 128.41 79.33) (end 127.26 78.18) (width 0.2) (layer "F.Cu") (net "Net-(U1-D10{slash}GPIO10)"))
 (segment (start 127.26 78.18) (end 107.755 78.18) (width 0.2) (layer "F.Cu") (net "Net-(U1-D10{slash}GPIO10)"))
 (segment (start 128.02 76.4) (end 116.725 76.4) (width 0.2) (layer "F.Cu") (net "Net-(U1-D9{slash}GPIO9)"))
 (segment (start 130.95 79.33) (end 128.02 76.4) (width 0.2) (layer "F.Cu") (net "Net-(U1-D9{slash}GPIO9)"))
 (segment (start 116.725 76.4) (end 111.25 70.925) (width 0.2) (layer "F.Cu") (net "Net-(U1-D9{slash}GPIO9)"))
 (segment (start 157.5 100) (end 160.08 102.58) (width 0.2) (layer "F.Cu") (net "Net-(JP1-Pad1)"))
 (segment (start 105.55 99.65) (end 105.55 104.55) (width 0.2) (layer "F.Cu") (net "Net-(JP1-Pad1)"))
 (segment (start 160.08 102.58) (end 166.5 102.58) (width 0.2) (layer "F.Cu") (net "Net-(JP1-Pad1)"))
 (segment (start 106 105) (end 147 105) (width 0.2) (layer "F.Cu") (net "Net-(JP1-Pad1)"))
 (segment (start 152 100) (end 157.5 100) (width 0.2) (layer "F.Cu") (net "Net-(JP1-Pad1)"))
 (segment (start 105.55 104.55) (end 106 105) (width 0.2) (layer "F.Cu") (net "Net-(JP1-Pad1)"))
 (segment (start 147 105) (end 152 100) (width 0.2) (layer "F.Cu") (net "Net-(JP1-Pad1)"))
 (segment (start 145.5 103) (end 130.5 103) (width 0.2) (layer "F.Cu") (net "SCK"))
 (segment (start 153.54 94.96) (end 145.5 103) (width 0.2) (layer "F.Cu") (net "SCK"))
 (segment (start 128.41 100.91) (end 128.41 99.65) (width 0.2) (layer "F.Cu") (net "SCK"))
 (segment (start 166.5 94.96) (end 153.54 94.96) (width 0.2) (layer "F.Cu") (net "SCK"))
 (segment (start 130.5 103) (end 128.41 100.91) (width 0.2) (layer "F.Cu") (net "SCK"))
 (segment (start 149.298377 92.42) (end 146.038377 95.68) (width 0.2) (layer "F.Cu") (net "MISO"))
 (segment (start 146.038377 95.68) (end 137.46 95.68) (width 0.2) (layer "F.Cu") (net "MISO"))
 (segment (start 137.46 95.68) (end 133.49 99.65) (width 0.2) (layer "F.Cu") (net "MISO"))
 (segment (start 166.5 92.42) (end 149.298377 92.42) (width 0.2) (layer "F.Cu") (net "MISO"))
 (segment (start 164.88 91.5) (end 148.5 91.5) (width 0.2) (layer "F.Cu") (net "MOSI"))
 (segment (start 136.1 94.5) (end 130.95 99.65) (width 0.2) (layer "F.Cu") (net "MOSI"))
 (segment (start 148.5 91.5) (end 145.5 94.5) (width 0.2) (layer "F.Cu") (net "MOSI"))
 (segment (start 166.5 89.88) (end 164.88 91.5) (width 0.2) (layer "F.Cu") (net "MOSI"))
 (segment (start 145.5 94.5) (end 136.1 94.5) (width 0.2) (layer "F.Cu") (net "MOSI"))
 (segment (start 151.5 84) (end 164.5 71) (width 0.2) (layer "F.Cu") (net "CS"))
 (segment (start 168 71) (end 170.5 73.5) (width 0.2) (layer "F.Cu") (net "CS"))
 (segment (start 170.5 73.5) (end 170.5 83.34) (width 0.2) (layer "F.Cu") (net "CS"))
 (segment (start 170.5 83.34) (end 166.5 87.34) (width 0.2) (layer "F.Cu") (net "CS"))
 (segment (start 125.87 79.33) (end 130.54 84) (width 0.2) (layer "F.Cu") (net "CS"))
 (segment (start 130.54 84) (end 151.5 84) (width 0.2) (layer "F.Cu") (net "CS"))
 (segment (start 164.5 71) (end 168 71) (width 0.2) (layer "F.Cu") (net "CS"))
 (segment (start 120.79 79.33) (end 127.96 86.5) (width 0.2) (layer "F.Cu") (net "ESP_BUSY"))
 (segment (start 164.8 86.5) (end 166.5 84.8) (width 0.2) (layer "F.Cu") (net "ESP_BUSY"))
 (segment (start 127.96 86.5) (end 164.8 86.5) (width 0.2) (layer "F.Cu") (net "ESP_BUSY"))
 (segment (start 129.5 85.5) (end 163.26 85.5) (width 0.2) (layer "F.Cu") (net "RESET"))
 (segment (start 163.26 85.5) (end 166.5 82.26) (width 0.2) (layer "F.Cu") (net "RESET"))
 (segment (start 123.33 79.33) (end 129.5 85.5) (width 0.2) (layer "F.Cu") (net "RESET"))
 (segment (start 133.49 79.33) (end 133.49 76.01) (width 0.2) (layer "F.Cu") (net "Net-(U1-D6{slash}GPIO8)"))
 (segment (start 133.49 76.01) (end 133.5 76) (width 0.2) (layer "F.Cu") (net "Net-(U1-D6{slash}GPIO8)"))
 (segment (start 127.075 76) (end 122 70.925) (width 0.2) (layer "F.Cu") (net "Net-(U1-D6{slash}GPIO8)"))
 (segment (start 133.5 76) (end 127.075 76) (width 0.2) (layer "F.Cu") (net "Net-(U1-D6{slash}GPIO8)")))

